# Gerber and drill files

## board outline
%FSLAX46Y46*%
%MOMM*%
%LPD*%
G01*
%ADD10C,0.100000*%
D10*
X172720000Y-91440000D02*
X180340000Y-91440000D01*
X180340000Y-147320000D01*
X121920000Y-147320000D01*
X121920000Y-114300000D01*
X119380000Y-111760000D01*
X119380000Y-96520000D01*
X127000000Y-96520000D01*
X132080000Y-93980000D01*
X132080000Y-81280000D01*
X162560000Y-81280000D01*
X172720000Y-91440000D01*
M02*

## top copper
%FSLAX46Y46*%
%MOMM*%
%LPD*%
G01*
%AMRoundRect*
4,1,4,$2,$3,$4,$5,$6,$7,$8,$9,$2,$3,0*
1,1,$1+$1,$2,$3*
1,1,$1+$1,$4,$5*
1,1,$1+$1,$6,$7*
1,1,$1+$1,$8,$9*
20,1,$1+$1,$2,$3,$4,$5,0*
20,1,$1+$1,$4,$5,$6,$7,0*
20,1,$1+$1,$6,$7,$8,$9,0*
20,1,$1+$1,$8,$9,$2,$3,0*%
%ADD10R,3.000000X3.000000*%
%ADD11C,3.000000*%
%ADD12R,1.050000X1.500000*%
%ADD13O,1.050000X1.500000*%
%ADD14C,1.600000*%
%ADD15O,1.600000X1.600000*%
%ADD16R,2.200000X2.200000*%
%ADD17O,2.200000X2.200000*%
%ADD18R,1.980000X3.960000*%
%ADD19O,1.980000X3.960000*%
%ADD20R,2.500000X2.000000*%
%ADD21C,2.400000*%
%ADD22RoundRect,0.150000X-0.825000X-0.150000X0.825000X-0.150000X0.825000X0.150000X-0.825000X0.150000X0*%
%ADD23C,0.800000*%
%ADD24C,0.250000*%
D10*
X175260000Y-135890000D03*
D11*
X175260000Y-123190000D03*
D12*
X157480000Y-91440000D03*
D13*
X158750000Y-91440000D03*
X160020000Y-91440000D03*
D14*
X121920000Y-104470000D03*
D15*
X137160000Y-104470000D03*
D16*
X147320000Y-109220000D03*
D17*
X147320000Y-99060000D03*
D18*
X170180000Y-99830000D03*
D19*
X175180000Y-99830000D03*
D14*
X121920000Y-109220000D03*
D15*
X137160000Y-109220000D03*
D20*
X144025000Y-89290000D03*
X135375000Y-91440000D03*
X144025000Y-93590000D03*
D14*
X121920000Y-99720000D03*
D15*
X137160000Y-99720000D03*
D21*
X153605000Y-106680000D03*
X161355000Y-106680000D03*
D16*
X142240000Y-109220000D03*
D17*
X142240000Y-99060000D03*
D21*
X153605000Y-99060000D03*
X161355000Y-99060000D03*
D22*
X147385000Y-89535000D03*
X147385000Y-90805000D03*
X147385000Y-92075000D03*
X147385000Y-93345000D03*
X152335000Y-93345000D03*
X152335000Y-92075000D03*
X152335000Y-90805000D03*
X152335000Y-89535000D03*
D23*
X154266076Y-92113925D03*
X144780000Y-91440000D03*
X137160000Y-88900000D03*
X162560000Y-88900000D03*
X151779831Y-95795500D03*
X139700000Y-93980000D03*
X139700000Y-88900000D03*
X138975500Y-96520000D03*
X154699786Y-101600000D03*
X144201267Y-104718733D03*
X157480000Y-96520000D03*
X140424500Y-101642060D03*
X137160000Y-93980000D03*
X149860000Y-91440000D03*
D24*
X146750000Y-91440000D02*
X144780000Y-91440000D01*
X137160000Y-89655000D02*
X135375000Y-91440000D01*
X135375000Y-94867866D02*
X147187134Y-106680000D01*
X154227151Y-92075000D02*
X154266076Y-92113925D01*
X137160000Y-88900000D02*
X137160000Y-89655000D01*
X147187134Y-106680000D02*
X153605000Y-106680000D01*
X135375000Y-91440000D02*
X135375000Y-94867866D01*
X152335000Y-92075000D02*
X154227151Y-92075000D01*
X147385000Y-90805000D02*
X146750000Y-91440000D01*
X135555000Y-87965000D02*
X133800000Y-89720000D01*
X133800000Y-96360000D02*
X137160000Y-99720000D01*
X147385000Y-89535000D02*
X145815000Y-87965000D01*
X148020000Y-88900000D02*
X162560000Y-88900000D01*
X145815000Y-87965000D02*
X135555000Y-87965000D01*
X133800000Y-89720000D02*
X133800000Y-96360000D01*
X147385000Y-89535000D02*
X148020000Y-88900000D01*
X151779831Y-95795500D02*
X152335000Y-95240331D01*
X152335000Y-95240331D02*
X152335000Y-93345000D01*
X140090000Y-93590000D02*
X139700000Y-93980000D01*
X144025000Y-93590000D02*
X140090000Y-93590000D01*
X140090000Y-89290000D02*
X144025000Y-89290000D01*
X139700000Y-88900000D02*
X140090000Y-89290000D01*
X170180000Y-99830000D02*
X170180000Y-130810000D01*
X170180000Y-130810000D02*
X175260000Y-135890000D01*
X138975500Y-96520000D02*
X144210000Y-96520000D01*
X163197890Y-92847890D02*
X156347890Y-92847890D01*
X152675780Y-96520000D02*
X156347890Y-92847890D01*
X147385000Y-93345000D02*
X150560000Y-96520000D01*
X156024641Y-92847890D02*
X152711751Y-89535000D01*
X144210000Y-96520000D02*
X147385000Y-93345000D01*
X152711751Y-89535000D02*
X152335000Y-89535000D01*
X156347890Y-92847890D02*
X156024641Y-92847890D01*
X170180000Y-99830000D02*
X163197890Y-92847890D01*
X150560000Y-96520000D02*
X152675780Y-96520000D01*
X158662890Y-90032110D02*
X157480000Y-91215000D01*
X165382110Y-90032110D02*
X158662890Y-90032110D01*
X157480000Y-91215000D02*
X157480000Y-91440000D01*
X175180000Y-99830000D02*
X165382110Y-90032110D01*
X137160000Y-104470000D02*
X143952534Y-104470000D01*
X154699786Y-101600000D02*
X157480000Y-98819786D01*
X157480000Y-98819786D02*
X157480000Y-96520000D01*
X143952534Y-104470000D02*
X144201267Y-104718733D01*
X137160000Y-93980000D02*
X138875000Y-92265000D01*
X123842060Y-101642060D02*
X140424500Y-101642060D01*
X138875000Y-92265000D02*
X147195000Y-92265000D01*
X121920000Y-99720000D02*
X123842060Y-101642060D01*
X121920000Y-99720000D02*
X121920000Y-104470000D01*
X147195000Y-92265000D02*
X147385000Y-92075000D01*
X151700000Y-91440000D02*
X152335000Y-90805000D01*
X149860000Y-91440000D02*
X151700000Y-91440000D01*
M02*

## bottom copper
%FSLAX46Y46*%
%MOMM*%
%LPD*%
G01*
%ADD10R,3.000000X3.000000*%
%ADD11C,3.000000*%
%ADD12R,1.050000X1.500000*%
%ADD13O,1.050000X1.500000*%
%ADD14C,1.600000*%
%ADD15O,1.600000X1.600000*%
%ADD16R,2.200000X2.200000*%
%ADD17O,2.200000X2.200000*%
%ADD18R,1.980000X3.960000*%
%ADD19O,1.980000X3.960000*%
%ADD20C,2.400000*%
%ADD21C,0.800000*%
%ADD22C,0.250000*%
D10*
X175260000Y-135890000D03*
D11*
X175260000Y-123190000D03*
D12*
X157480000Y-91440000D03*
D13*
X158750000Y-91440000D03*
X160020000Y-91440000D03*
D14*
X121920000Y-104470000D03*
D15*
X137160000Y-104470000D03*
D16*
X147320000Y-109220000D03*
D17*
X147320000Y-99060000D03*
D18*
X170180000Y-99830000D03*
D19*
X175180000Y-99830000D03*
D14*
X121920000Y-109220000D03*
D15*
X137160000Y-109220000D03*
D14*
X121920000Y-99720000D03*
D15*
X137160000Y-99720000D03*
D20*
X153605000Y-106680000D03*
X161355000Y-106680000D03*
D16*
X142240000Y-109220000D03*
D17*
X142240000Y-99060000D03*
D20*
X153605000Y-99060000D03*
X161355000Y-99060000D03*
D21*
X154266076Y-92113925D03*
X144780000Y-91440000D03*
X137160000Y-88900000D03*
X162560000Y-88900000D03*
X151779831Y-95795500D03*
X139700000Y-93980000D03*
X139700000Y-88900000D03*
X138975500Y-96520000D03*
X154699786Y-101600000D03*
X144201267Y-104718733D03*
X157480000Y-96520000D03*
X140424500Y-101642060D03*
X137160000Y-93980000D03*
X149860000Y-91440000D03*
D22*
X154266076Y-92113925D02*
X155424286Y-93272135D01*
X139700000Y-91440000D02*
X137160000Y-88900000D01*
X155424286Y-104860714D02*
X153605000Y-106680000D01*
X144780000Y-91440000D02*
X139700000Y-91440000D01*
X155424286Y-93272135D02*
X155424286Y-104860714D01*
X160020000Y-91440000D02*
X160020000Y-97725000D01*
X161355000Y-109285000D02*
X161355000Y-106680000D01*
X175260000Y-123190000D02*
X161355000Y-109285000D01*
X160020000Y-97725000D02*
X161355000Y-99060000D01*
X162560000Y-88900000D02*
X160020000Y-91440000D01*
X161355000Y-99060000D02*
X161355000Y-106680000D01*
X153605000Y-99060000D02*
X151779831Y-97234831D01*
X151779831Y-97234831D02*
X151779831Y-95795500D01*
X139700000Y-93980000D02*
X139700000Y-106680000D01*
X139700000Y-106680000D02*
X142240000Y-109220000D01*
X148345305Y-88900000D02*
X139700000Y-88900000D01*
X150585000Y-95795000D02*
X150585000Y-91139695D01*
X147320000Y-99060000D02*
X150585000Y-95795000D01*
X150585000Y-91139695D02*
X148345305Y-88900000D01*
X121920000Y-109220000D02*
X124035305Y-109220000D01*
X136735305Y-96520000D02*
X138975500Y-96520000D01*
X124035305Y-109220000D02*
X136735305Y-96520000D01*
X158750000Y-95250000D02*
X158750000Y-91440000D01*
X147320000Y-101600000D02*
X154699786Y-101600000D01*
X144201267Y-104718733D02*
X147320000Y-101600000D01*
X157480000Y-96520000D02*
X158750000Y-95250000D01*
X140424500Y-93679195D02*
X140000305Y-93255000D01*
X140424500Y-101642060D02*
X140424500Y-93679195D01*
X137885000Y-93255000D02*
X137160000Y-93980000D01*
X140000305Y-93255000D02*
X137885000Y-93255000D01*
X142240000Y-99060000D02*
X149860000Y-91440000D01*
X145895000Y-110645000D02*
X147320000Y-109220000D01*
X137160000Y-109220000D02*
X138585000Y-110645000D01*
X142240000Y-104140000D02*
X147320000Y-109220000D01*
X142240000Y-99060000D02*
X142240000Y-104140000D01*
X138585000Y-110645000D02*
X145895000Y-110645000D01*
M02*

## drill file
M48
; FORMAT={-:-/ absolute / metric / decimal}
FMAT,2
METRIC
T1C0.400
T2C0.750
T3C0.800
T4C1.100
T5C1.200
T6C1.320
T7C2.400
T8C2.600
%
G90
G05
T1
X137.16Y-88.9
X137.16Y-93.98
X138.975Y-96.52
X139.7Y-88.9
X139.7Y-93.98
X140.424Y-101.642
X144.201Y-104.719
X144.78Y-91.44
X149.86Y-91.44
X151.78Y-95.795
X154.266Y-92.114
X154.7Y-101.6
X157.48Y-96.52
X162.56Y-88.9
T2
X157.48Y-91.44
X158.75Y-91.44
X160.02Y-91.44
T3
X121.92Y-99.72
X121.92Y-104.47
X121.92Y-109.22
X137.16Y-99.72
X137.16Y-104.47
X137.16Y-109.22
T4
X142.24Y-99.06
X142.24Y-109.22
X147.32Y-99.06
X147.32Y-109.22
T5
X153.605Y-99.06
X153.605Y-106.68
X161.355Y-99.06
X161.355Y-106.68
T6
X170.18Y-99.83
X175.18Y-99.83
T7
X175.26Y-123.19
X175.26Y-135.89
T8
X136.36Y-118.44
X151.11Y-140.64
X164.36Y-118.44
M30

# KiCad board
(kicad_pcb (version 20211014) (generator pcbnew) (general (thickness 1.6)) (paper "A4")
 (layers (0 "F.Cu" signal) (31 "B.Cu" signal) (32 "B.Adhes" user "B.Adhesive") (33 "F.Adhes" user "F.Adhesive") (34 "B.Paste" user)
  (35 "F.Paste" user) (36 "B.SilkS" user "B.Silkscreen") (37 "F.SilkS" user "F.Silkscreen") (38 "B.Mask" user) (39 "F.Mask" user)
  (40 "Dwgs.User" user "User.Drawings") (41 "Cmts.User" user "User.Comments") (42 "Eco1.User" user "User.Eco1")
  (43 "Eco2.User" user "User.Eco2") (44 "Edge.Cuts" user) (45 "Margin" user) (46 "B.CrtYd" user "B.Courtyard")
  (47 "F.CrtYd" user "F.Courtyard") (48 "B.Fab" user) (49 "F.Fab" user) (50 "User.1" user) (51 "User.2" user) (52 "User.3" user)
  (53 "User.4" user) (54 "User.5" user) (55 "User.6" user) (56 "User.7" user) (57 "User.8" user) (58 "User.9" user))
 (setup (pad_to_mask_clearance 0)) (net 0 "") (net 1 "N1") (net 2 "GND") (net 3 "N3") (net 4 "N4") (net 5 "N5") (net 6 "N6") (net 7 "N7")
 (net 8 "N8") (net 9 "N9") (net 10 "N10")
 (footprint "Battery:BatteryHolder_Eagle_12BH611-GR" (layer "F.Cu") (at 175.26 135.89)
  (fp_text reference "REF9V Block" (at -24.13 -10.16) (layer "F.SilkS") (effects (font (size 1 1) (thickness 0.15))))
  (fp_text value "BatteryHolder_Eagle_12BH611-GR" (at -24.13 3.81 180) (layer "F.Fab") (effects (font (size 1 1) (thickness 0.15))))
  (pad "" np_thru_hole circle (at -38.9 -17.45) (size 2.6 2.6) (drill 2.6) (layers *.Cu *.Mask))
  (pad "" np_thru_hole circle (at -24.15 4.75) (size 2.6 2.6) (drill 2.6) (layers *.Cu *.Mask))
  (pad "" np_thru_hole circle (at -10.9 -17.45) (size 2.6 2.6) (drill 2.6) (layers *.Cu *.Mask))
  (pad "1" thru_hole rect (at 0 0) (size 3 3) (drill 2.4) (layers *.Cu *.Mask) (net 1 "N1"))
  (pad "2" thru_hole circle (at 0 -12.7) (size 3 3) (drill 2.4) (layers *.Cu *.Mask) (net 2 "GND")))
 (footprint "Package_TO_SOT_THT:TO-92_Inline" (layer "F.Cu") (at 157.48 91.44)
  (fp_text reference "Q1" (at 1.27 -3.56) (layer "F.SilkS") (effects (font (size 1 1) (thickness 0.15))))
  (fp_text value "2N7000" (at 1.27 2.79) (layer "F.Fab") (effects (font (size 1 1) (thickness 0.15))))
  (pad "1" thru_hole rect (at 0 0) (size 1.05 1.5) (drill 0.75) (layers *.Cu *.Mask) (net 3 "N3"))
  (pad "2" thru_hole oval (at 1.27 0) (size 1.05 1.5) (drill 0.75) (layers *.Cu *.Mask) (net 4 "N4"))
  (pad "3" thru_hole oval (at 2.54 0) (size 1.05 1.5) (drill 0.75) (layers *.Cu *.Mask) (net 2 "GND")))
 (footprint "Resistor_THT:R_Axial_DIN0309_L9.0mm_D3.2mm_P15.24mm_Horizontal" (layer "F.Cu") (at 121.92 104.47)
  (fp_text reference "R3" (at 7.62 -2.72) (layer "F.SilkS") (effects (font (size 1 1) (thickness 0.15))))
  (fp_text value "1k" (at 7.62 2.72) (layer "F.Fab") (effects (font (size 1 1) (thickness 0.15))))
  (pad "1" thru_hole circle (at 0 0) (size 1.6 1.6) (drill 0.8) (layers *.Cu *.Mask) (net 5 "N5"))
  (pad "2" thru_hole oval (at 15.24 0) (size 1.6 1.6) (drill 0.8) (layers *.Cu *.Mask) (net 4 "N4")))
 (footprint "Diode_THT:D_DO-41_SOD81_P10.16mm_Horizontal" (layer "F.Cu") (at 147.32 109.22 90)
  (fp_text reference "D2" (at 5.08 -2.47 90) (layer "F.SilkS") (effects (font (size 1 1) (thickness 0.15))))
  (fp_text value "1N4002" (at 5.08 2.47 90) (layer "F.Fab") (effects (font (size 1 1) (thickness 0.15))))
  (pad "1" thru_hole rect (at 0 0 90) (size 2.2 2.2) (drill 1.1) (layers *.Cu *.Mask) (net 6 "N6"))
  (pad "2" thru_hole oval (at 10.16 0 90) (size 2.2 2.2) (drill 1.1) (layers *.Cu *.Mask) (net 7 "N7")))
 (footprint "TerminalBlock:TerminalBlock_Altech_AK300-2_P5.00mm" (layer "F.Cu") (at 170.18 99.83)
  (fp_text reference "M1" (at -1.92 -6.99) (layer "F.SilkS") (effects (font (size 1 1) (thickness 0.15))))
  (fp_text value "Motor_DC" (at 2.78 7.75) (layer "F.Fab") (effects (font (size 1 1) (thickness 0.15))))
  (pad "1" thru_hole rect (at 0 0) (size 1.98 3.96) (drill 1.32) (layers *.Cu *.Mask) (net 1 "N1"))
  (pad "2" thru_hole oval (at 5 0) (size 1.98 3.96) (drill 1.32) (layers *.Cu *.Mask) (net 3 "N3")))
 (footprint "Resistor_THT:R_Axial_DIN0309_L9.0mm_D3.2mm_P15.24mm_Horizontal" (layer "F.Cu") (at 121.92 109.22)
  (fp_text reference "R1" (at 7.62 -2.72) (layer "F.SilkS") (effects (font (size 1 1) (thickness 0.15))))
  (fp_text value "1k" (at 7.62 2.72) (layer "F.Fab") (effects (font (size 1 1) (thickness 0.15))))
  (pad "1" thru_hole circle (at 0 0) (size 1.6 1.6) (drill 0.8) (layers *.Cu *.Mask) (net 1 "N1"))
  (pad "2" thru_hole oval (at 15.24 0) (size 1.6 1.6) (drill 0.8) (layers *.Cu *.Mask) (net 6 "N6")))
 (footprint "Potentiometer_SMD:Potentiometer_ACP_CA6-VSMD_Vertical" (layer "F.Cu") (at 139.7 91.44 180)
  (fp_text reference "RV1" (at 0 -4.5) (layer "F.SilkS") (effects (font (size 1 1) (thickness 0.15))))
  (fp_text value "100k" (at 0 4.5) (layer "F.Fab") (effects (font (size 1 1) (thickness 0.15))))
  (pad "1" smd rect (at -4.325 2.15 180) (size 2.5 2) (layers "F.Cu" "F.Paste" "F.Mask") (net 7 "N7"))
  (pad "2" smd rect (at 4.325 0 180) (size 2.5 2) (layers "F.Cu" "F.Paste" "F.Mask") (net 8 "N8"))
  (pad "3" smd rect (at -4.325 -2.15 180) (size 2.5 2) (layers "F.Cu" "F.Paste" "F.Mask") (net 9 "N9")))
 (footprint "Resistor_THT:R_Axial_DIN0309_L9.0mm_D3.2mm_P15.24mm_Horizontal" (layer "F.Cu") (at 121.92 99.72)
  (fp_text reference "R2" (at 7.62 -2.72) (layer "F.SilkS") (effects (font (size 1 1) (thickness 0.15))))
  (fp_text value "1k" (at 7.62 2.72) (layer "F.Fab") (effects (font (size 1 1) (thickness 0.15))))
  (pad "1" thru_hole circle (at 0 0) (size 1.6 1.6) (drill 0.8) (layers *.Cu *.Mask) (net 5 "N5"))
  (pad "2" thru_hole oval (at 15.24 0) (size 1.6 1.6) (drill 0.8) (layers *.Cu *.Mask) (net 2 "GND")))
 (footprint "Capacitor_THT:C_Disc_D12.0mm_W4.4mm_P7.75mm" (layer "F.Cu") (at 153.605 106.68)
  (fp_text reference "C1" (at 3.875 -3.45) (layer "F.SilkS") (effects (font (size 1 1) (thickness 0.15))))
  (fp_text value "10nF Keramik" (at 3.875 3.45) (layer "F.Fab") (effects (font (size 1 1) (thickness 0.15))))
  (pad "1" thru_hole circle (at 0 0) (size 2.4 2.4) (drill 1.2) (layers *.Cu *.Mask) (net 8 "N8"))
  (pad "2" thru_hole circle (at 7.75 0) (size 2.4 2.4) (drill 1.2) (layers *.Cu *.Mask) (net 2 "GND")))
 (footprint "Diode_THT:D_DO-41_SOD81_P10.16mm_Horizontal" (layer "F.Cu") (at 142.24 109.22 90)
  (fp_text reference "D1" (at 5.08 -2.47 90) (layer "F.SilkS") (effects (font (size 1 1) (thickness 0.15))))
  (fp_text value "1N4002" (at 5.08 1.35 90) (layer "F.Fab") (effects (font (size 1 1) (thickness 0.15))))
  (pad "1" thru_hole rect (at 0 0 90) (size 2.2 2.2) (drill 1.1) (layers *.Cu *.Mask) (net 9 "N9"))
  (pad "2" thru_hole oval (at 10.16 0 90) (size 2.2 2.2) (drill 1.1) (layers *.Cu *.Mask) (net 6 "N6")))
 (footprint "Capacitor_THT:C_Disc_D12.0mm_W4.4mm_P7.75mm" (layer "F.Cu") (at 153.605 99.06)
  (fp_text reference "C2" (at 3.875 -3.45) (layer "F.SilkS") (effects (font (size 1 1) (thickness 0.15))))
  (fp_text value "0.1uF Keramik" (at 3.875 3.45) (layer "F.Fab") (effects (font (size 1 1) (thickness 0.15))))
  (pad "1" thru_hole circle (at 0 0) (size 2.4 2.4) (drill 1.2) (layers *.Cu *.Mask) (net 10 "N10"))
  (pad "2" thru_hole circle (at 7.75 0) (size 2.4 2.4) (drill 1.2) (layers *.Cu *.Mask) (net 2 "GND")))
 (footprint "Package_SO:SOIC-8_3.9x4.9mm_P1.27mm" (layer "F.Cu") (at 149.86 91.44)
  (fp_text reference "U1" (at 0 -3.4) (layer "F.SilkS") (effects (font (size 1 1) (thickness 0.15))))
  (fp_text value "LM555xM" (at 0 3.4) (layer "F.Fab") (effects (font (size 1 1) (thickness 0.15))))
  (pad "1" smd roundrect (at -2.475 -1.905) (size 1.95 0.6) (layers "F.Cu" "F.Paste" "F.Mask") (roundrect_rratio 0.25) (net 2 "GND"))
  (pad "2" smd roundrect (at -2.475 -0.635) (size 1.95 0.6) (layers "F.Cu" "F.Paste" "F.Mask") (roundrect_rratio 0.25) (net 8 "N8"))
  (pad "3" smd roundrect (at -2.475 0.635) (size 1.95 0.6) (layers "F.Cu" "F.Paste" "F.Mask") (roundrect_rratio 0.25) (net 5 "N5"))
  (pad "4" smd roundrect (at -2.475 1.905) (size 1.95 0.6) (layers "F.Cu" "F.Paste" "F.Mask") (roundrect_rratio 0.25) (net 1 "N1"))
  (pad "5" smd roundrect (at 2.475 1.905) (size 1.95 0.6) (layers "F.Cu" "F.Paste" "F.Mask") (roundrect_rratio 0.25) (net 10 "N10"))
  (pad "6" smd roundrect (at 2.475 0.635) (size 1.95 0.6) (layers "F.Cu" "F.Paste" "F.Mask") (roundrect_rratio 0.25) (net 8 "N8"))
  (pad "7" smd roundrect (at 2.475 -0.635) (size 1.95 0.6) (layers "F.Cu" "F.Paste" "F.Mask") (roundrect_rratio 0.25) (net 6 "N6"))
  (pad "8" smd roundrect (at 2.475 -1.905) (size 1.95 0.6) (layers "F.Cu" "F.Paste" "F.Mask") (roundrect_rratio 0.25) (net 1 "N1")))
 (gr_poly
  (pts (xy 172.72 91.44) (xy 180.34 91.44) (xy 180.34 147.32) (xy 121.92 147.32) (xy 121.92 114.3) (xy 119.38 111.76) (xy 119.38 96.52)
   (xy 127 96.52) (xy 132.08 93.98) (xy 132.08 81.28) (xy 162.56 81.28))
  (layer "Edge.Cuts") (width 0.1) (fill none))
 (segment (start 146.75 91.44) (end 144.78 91.44) (width 0.25) (layer "F.Cu") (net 8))
 (segment (start 137.16 89.655) (end 135.375 91.44) (width 0.25) (layer "F.Cu") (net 8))
 (segment (start 135.375 94.867866) (end 147.187134 106.68) (width 0.25) (layer "F.Cu") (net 8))
 (segment (start 154.227151 92.075) (end 154.266076 92.113925) (width 0.25) (layer "F.Cu") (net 8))
 (segment (start 137.16 88.9) (end 137.16 89.655) (width 0.25) (layer "F.Cu") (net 8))
 (segment (start 147.187134 106.68) (end 153.605 106.68) (width 0.25) (layer "F.Cu") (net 8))
 (segment (start 135.375 91.44) (end 135.375 94.867866) (width 0.25) (layer "F.Cu") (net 8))
 (segment (start 152.335 92.075) (end 154.227151 92.075) (width 0.25) (layer "F.Cu") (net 8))
 (segment (start 147.385 90.805) (end 146.75 91.44) (width 0.25) (layer "F.Cu") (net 8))
 (via (at 154.266076 92.113925) (size 0.8) (drill 0.4) (layers "F.Cu" "B.Cu") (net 8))
 (via (at 144.78 91.44) (size 0.8) (drill 0.4) (layers "F.Cu" "B.Cu") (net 8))
 (via (at 137.16 88.9) (size 0.8) (drill 0.4) (layers "F.Cu" "B.Cu") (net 8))
 (segment (start 154.266076 92.113925) (end 155.424286 93.272135) (width 0.25) (layer "B.Cu") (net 8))
 (segment (start 139.7 91.44) (end 137.16 88.9) (width 0.25) (layer "B.Cu") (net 8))
 (segment (start 155.424286 104.860714) (end 153.605 106.68) (width 0.25) (layer "B.Cu") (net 8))
 (segment (start 144.78 91.44) (end 139.7 91.44) (width 0.25) (layer "B.Cu") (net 8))
 (segment (start 155.424286 93.272135) (end 155.424286 104.860714) (width 0.25) (layer "B.Cu") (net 8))
 (segment (start 135.555 87.965) (end 133.8 89.72) (width 0.25) (layer "F.Cu") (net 2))
 (segment (start 133.8 96.36) (end 137.16 99.72) (width 0.25) (layer "F.Cu") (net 2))
 (segment (start 147.385 89.535) (end 145.815 87.965) (width 0.25) (layer "F.Cu") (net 2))
 (segment (start 148.02 88.9) (end 162.56 88.9) (width 0.25) (layer "F.Cu") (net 2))
 (segment (start 145.815 87.965) (end 135.555 87.965) (width 0.25) (layer "F.Cu") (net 2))
 (segment (start 133.8 89.72) (end 133.8 96.36) (width 0.25) (layer "F.Cu") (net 2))
 (segment (start 147.385 89.535) (end 148.02 88.9) (width 0.25) (layer "F.Cu") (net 2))
 (via (at 162.56 88.9) (size 0.8) (drill 0.4) (layers "F.Cu" "B.Cu") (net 2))
 (segment (start 160.02 91.44) (end 160.02 97.725) (width 0.25) (layer "B.Cu") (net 2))
 (segment (start 161.355 109.285) (end 161.355 106.68) (width 0.25) (layer "B.Cu") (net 2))
 (segment (start 175.26 123.19) (end 161.355 109.285) (width 0.25) (layer "B.Cu") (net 2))
 (segment (start 160.02 97.725) (end 161.355 99.06) (width 0.25) (layer "B.Cu") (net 2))
 (segment (start 162.56 88.9) (end 160.02 91.44) (width 0.25) (layer "B.Cu") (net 2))
 (segment (start 161.355 99.06) (end 161.355 106.68) (width 0.25) (layer "B.Cu") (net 2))
 (segment (start 151.779831 95.7955) (end 152.335 95.240331) (width 0.25) (layer "F.Cu") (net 10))
 (segment (start 152.335 95.240331) (end 152.335 93.345) (width 0.25) (layer "F.Cu") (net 10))
 (via (at 151.779831 95.7955) (size 0.8) (drill 0.4) (layers "F.Cu" "B.Cu") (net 10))
 (segment (start 153.605 99.06) (end 151.779831 97.234831) (width 0.25) (layer "B.Cu") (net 10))
 (segment (start 151.779831 97.234831) (end 151.779831 95.7955) (width 0.25) (layer "B.Cu") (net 10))
 (segment (start 140.09 93.59) (end 139.7 93.98) (width 0.25) (layer "F.Cu") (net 9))
 (segment (start 144.025 93.59) (end 140.09 93.59) (width 0.25) (layer "F.Cu") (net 9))
 (via (at 139.7 93.98) (size 0.8) (drill 0.4) (layers "F.Cu" "B.Cu") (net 9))
 (segment (start 139.7 93.98) (end 139.7 106.68) (width 0.25) (layer "B.Cu") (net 9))
 (segment (start 139.7 106.68) (end 142.24 109.22) (width 0.25) (layer "B.Cu") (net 9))
 (segment (start 140.09 89.29) (end 144.025 89.29) (width 0.25) (layer "F.Cu") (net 7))
 (segment (start 139.7 88.9) (end 140.09 89.29) (width 0.25) (layer "F.Cu") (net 7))
 (via (at 139.7 88.9) (size 0.8) (drill 0.4) (layers "F.Cu" "B.Cu") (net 7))
 (segment (start 148.345305 88.9) (end 139.7 88.9) (width 0.25) (layer "B.Cu") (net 7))
 (segment (start 150.585 95.795) (end 150.585 91.139695) (width 0.25) (layer "B.Cu") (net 7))
 (segment (start 147.32 99.06) (end 150.585 95.795) (width 0.25) (layer "B.Cu") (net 7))
 (segment (start 150.585 91.139695) (end 148.345305 88.9) (width 0.25) (layer "B.Cu") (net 7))
 (segment (start 170.18 99.83) (end 170.18 130.81) (width 0.25) (layer "F.Cu") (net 1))
 (segment (start 170.18 130.81) (end 175.26 135.89) (width 0.25) (layer "F.Cu") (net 1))
 (segment (start 138.9755 96.52) (end 144.21 96.52) (width 0.25) (layer "F.Cu") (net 1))
 (segment (start 163.19789 92.84789) (end 156.34789 92.84789) (width 0.25) (layer "F.Cu") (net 1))
 (segment (start 152.67578 96.52) (end 156.34789 92.84789) (width 0.25) (layer "F.Cu") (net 1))
 (segment (start 147.385 93.345) (end 150.56 96.52) (width 0.25) (layer "F.Cu") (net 1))
 (segment (start 156.024641 92.84789) (end 152.711751 89.535) (width 0.25) (layer "F.Cu") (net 1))
 (segment (start 144.21 96.52) (end 147.385 93.345) (width 0.25) (layer "F.Cu") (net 1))
 (segment (start 152.711751 89.535) (end 152.335 89.535) (width 0.25) (layer "F.Cu") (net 1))
 (segment (start 156.34789 92.84789) (end 156.024641 92.84789) (width 0.25) (layer "F.Cu") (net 1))
 (segment (start 170.18 99.83) (end 163.19789 92.84789) (width 0.25) (layer "F.Cu") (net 1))
 (segment (start 150.56 96.52) (end 152.67578 96.52) (width 0.25) (layer "F.Cu") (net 1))
 (via (at 138.9755 96.52) (size 0.8) (drill 0.4) (layers "F.Cu" "B.Cu") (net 1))
 (segment (start 121.92 109.22) (end 124.035305 109.22) (width 0.25) (layer "B.Cu") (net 1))
 (segment (start 136.735305 96.52) (end 138.9755 96.52) (width 0.25) (layer "B.Cu") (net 1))
 (segment (start 124.035305 109.22) (end 136.735305 96.52) (width 0.25) (layer "B.Cu") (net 1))
 (segment (start 158.66289 90.03211) (end 157.48 91.215) (width 0.25) (layer "F.Cu") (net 3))
 (segment (start 165.38211 90.03211) (end 158.66289 90.03211) (width 0.25) (layer "F.Cu") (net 3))
 (segment (start 157.48 91.215) (end 157.48 91.44) (width 0.25) (layer "F.Cu") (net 3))
 (segment (start 175.18 99.83) (end 165.38211 90.03211) (width 0.25) (layer "F.Cu") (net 3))
 (segment (start 137.16 104.47) (end 143.952534 104.47) (width 0.25) (layer "F.Cu") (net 4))
 (segment (start 154.699786 101.6) (end 157.48 98.819786) (width 0.25) (layer "F.Cu") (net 4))
 (segment (start 157.48 98.819786) (end 157.48 96.52) (width 0.25) (layer "F.Cu") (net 4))
 (segment (start 143.952534 104.47) (end 144.201267 104.718733) (width 0.25) (layer "F.Cu") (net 4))
 (via (at 154.699786 101.6) (size 0.8) (drill 0.4) (layers "F.Cu" "B.Cu") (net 4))
 (via (at 144.201267 104.718733) (size 0.8) (drill 0.4) (layers "F.Cu" "B.Cu") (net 4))
 (via (at 157.48 96.52) (size 0.8) (drill 0.4) (layers "F.Cu" "B.Cu") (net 4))
 (segment (start 158.75 95.25) (end 158.75 91.44) (width 0.25) (layer "B.Cu") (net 4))
 (segment (start 147.32 101.6) (end 154.699786 101.6) (width 0.25) (layer "B.Cu") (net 4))
 (segment (start 144.201267 104.718733) (end 147.32 101.6) (width 0.25) (layer "B.Cu") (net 4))
 (segment (start 157.48 96.52) (end 158.75 95.25) (width 0.25) (layer "B.Cu") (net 4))
 (segment (start 137.16 93.98) (end 138.875 92.265) (width 0.25) (layer "F.Cu") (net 5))
 (segment (start 123.84206 101.64206) (end 140.4245 101.64206) (width 0.25) (layer "F.Cu") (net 5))
 (segment (start 138.875 92.265) (end 147.195 92.265) (width 0.25) (layer "F.Cu") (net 5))
 (segment (start 121.92 99.72) (end 123.84206 101.64206) (width 0.25) (layer "F.Cu") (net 5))
 (segment (start 121.92 99.72) (end 121.92 104.47) (width 0.25) (layer "F.Cu") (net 5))
 (segment (start 147.195 92.265) (end 147.385 92.075) (width 0.25) (layer "F.Cu") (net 5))
 (via (at 140.4245 101.64206) (size 0.8) (drill 0.4) (layers "F.Cu" "B.Cu") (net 5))
 (via (at 137.16 93.98) (size 0.8) (drill 0.4) (layers "F.Cu" "B.Cu") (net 5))
 (segment (start 140.4245 93.679195) (end 140.000305 93.255) (width 0.25) (layer "B.Cu") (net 5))
 (segment (start 140.4245 101.64206) (end 140.4245 93.679195) (width 0.25) (layer "B.Cu") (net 5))
 (segment (start 137.885 93.255) (end 137.16 93.98) (width 0.25) (layer "B.Cu") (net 5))
 (segment (start 140.000305 93.255) (end 137.885 93.255) (width 0.25) (layer "B.Cu") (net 5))
 (segment (start 151.7 91.44) (end 152.335 90.805) (width 0.25) (layer "F.Cu") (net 6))
 (segment (start 149.86 91.44) (end 151.7 91.44) (width 0.25) (layer "F.Cu") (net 6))
 (via (at 149.86 91.44) (size 0.8) (drill 0.4) (layers "F.Cu" "B.Cu") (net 6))
 (segment (start 142.24 99.06) (end 149.86 91.44) (width 0.25) (layer "B.Cu") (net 6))
 (segment (start 145.895 110.645) (end 147.32 109.22) (width 0.25) (layer "B.Cu") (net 6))
 (segment (start 137.16 109.22) (end 138.585 110.645) (width 0.25) (layer "B.Cu") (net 6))
 (segment (start 142.24 104.14) (end 147.32 109.22) (width 0.25) (layer "B.Cu") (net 6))
 (segment (start 142.24 99.06) (end 142.24 104.14) (width 0.25) (layer "B.Cu") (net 6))
 (segment (start 138.585 110.645) (end 145.895 110.645) (width 0.25) (layer "B.Cu") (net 6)))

